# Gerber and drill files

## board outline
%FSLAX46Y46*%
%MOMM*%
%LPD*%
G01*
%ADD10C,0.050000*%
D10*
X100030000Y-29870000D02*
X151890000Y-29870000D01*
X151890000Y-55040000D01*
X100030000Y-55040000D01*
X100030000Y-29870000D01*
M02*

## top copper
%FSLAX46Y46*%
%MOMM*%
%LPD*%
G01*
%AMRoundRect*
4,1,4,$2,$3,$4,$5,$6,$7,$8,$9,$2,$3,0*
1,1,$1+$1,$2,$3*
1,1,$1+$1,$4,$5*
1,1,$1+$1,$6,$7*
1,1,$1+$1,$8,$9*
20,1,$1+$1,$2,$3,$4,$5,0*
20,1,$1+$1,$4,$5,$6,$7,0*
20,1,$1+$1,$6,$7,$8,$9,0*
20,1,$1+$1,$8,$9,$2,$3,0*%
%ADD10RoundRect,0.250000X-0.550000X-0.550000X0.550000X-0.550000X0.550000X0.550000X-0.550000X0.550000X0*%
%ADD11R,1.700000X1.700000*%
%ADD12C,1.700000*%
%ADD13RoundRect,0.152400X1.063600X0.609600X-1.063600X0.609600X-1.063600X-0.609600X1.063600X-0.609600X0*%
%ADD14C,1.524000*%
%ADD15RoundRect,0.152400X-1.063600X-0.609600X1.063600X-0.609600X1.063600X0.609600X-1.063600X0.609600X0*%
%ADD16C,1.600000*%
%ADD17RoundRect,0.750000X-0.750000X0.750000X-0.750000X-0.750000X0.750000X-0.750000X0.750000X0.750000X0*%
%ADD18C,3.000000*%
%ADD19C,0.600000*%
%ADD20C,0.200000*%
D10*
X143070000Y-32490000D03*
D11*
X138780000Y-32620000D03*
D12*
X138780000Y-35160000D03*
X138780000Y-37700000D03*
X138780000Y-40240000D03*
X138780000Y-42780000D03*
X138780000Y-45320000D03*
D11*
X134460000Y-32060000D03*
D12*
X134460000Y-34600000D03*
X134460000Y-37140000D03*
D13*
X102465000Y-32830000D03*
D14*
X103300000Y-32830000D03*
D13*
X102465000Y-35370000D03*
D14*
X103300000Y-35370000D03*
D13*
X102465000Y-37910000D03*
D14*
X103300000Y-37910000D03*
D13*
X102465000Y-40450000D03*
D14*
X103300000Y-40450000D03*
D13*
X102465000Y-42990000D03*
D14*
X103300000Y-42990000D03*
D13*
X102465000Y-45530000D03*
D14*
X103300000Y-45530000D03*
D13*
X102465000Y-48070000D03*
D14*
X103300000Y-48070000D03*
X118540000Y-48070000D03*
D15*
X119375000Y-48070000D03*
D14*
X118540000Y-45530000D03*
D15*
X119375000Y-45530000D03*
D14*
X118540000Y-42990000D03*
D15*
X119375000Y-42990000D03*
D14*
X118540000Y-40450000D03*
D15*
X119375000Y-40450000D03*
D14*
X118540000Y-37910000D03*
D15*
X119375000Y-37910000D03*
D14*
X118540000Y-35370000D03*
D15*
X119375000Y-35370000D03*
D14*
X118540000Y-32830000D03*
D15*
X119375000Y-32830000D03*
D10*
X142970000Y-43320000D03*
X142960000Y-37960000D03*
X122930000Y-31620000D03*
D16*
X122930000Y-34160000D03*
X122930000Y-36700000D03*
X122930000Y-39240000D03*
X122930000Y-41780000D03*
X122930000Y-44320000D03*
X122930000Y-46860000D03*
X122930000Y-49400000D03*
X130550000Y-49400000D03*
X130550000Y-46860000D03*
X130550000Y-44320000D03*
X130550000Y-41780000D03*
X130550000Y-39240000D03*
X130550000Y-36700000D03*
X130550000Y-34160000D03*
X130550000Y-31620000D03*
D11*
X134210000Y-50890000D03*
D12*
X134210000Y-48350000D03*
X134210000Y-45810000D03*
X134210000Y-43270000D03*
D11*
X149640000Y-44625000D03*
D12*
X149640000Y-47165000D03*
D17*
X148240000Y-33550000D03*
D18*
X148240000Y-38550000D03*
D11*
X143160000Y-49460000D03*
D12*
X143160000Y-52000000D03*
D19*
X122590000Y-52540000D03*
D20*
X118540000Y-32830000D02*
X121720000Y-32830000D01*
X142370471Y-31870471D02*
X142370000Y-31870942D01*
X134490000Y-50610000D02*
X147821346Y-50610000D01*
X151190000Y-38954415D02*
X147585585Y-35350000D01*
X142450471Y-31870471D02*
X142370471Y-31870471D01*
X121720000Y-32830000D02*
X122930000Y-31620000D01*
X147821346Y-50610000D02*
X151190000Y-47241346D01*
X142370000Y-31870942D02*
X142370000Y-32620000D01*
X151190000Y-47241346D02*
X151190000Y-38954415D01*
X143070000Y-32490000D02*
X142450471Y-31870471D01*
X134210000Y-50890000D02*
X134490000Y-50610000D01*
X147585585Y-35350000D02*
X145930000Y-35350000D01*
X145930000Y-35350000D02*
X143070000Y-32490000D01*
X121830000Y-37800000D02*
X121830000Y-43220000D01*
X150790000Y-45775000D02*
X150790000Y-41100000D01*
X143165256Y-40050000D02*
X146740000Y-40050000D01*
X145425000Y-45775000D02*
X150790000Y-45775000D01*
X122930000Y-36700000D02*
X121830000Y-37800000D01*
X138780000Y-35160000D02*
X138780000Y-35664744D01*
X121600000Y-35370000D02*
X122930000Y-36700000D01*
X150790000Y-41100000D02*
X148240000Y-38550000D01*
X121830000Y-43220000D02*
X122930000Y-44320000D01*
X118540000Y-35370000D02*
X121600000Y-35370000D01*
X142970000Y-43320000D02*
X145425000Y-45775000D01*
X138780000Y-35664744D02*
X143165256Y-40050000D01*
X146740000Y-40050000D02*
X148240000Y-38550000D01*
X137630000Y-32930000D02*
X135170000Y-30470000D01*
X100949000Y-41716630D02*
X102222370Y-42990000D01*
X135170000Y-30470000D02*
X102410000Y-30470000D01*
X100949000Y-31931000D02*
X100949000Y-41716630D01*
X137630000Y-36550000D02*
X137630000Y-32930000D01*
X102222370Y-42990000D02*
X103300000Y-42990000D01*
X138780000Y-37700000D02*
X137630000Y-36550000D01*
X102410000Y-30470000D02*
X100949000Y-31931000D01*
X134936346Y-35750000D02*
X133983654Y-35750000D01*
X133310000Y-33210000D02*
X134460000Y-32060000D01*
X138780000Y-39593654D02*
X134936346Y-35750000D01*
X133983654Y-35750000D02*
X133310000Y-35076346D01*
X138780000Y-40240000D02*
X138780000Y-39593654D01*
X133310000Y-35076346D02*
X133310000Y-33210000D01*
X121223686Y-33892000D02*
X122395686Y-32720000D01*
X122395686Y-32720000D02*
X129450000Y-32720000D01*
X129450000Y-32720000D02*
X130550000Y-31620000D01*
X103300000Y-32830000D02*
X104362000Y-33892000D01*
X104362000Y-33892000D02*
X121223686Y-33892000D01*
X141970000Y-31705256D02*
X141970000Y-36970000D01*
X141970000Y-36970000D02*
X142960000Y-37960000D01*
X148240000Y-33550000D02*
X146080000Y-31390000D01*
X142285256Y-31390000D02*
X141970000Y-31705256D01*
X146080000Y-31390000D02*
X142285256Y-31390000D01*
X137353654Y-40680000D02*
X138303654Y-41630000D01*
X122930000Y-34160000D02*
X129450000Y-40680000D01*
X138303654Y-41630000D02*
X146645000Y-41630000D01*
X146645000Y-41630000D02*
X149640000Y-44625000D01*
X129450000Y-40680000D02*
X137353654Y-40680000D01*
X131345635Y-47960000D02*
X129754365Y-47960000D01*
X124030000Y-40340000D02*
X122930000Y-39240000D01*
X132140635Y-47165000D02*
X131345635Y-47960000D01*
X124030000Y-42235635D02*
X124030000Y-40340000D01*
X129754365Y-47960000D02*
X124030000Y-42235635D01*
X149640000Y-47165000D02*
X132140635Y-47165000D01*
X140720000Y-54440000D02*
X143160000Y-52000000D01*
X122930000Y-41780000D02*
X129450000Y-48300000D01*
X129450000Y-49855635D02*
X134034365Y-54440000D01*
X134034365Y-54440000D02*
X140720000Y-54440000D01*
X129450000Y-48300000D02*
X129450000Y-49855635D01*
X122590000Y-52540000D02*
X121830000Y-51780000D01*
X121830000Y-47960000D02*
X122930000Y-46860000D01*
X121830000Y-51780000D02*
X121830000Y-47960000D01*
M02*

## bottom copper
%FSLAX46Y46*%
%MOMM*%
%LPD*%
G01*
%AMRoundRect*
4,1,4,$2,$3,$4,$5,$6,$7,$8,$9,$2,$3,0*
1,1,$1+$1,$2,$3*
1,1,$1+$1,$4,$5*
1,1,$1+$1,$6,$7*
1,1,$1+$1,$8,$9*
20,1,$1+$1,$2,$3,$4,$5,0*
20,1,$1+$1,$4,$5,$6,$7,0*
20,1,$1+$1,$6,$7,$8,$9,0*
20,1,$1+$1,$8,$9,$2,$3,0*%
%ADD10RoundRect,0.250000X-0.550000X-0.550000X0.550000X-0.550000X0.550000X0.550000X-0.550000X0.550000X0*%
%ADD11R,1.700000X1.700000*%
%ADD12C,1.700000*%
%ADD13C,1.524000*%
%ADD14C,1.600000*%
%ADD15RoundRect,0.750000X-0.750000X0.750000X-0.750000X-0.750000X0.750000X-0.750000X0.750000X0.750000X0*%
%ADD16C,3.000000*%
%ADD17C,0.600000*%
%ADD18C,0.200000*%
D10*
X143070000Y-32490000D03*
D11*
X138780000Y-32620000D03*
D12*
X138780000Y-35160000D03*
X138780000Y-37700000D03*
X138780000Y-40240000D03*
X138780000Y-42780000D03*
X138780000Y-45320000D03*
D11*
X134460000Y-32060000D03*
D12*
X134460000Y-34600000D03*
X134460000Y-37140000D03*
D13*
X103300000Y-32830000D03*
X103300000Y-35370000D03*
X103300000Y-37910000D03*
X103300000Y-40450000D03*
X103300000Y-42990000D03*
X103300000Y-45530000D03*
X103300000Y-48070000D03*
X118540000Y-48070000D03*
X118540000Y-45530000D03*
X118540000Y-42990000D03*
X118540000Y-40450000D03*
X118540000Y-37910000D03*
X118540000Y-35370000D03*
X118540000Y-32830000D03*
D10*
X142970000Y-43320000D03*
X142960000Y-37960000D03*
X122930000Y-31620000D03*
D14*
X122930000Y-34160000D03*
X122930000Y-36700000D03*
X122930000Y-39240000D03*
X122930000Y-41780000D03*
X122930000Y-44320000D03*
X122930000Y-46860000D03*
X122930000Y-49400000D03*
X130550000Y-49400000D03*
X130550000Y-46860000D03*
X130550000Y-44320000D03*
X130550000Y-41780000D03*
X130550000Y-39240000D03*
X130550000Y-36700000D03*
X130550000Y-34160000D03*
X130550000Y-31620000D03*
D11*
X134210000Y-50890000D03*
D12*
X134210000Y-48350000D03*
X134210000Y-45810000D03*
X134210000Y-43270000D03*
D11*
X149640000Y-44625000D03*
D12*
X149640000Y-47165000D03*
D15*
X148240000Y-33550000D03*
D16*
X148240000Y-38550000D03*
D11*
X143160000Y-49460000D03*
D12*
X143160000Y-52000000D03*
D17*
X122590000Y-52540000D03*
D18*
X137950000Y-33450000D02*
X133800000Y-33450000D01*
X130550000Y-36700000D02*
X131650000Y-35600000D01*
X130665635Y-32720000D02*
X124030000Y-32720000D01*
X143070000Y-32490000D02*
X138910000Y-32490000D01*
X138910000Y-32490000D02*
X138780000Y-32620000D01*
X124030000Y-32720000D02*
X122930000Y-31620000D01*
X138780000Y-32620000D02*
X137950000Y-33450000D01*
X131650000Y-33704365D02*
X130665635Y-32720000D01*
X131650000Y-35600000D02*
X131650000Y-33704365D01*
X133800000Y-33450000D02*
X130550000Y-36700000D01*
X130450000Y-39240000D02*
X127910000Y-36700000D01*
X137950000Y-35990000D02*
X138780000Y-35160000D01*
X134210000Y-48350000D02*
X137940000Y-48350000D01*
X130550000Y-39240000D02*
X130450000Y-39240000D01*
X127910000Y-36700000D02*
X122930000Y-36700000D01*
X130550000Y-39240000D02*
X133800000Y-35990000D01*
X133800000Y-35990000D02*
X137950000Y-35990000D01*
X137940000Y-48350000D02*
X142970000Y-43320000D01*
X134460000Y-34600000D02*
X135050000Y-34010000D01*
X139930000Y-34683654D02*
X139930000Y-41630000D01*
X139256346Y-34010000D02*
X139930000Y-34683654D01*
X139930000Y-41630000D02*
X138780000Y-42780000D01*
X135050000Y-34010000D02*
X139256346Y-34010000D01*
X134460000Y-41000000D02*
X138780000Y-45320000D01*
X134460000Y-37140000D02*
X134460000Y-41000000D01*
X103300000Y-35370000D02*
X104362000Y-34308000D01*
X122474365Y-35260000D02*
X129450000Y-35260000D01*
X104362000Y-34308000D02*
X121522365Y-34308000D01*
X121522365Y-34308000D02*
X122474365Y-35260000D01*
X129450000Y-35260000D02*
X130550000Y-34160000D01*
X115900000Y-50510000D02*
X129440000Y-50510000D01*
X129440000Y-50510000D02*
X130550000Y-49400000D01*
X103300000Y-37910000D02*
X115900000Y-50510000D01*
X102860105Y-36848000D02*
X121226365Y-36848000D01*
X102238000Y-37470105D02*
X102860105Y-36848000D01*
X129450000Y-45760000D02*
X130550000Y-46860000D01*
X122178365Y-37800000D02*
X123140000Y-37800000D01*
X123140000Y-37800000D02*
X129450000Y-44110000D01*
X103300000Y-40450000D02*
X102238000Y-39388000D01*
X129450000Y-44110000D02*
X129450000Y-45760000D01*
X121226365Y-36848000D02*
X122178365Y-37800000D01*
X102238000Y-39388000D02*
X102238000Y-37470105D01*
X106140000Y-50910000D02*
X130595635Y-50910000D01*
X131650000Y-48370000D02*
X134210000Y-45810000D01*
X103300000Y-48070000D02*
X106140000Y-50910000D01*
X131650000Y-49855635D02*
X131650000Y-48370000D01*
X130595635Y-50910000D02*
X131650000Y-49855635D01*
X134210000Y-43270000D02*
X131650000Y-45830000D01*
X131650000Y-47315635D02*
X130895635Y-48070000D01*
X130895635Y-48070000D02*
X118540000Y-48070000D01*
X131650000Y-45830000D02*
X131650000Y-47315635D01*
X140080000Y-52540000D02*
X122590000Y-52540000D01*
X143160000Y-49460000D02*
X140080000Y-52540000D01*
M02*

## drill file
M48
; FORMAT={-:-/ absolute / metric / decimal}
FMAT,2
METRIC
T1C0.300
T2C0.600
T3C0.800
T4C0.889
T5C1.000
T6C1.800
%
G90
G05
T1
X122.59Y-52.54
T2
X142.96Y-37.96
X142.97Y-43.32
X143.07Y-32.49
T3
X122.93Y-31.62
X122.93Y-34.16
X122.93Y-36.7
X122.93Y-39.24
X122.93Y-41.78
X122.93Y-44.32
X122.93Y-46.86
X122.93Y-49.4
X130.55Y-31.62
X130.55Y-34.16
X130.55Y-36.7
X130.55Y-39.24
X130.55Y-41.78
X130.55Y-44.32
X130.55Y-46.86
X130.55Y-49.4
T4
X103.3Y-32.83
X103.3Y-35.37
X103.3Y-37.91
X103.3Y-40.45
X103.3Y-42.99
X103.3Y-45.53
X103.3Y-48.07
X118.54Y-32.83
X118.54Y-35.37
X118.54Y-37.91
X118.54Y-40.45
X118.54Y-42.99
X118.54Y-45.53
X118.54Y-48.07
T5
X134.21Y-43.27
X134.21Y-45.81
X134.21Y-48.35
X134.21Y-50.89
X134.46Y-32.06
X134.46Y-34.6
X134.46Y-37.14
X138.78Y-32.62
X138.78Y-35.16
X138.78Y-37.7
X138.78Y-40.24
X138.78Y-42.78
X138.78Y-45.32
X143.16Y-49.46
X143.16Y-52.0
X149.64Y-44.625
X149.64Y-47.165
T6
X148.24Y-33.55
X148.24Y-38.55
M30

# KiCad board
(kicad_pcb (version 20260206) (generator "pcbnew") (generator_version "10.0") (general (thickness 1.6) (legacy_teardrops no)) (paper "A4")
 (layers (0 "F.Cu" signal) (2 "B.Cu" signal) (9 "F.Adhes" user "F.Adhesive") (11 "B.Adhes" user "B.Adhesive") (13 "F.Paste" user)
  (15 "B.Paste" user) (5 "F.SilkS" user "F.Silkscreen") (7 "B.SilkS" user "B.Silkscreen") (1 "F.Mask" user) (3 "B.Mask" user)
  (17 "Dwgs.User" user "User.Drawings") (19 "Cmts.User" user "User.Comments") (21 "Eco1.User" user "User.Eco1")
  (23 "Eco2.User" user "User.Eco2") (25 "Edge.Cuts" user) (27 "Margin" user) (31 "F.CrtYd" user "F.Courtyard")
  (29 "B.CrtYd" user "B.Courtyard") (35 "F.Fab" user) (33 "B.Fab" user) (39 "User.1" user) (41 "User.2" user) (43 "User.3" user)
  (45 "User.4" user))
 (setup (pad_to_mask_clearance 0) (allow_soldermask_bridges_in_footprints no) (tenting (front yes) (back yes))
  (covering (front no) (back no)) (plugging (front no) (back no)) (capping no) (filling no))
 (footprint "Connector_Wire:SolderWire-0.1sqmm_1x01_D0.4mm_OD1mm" (layer "F.Cu") (at 143.07 32.49)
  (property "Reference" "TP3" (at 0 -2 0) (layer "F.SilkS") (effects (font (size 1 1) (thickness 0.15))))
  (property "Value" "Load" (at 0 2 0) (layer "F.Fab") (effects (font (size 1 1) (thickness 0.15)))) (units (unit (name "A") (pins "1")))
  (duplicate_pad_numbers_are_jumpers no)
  (pad "1" thru_hole roundrect (at 0 0) (size 1.6 1.6) (drill 0.6) (layers "*.Cu" "*.Mask") (remove_unused_layers no)
   (roundrect_rratio 0.15625) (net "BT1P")))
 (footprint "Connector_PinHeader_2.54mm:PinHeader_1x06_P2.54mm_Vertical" (layer "F.Cu") (at 138.78 32.62)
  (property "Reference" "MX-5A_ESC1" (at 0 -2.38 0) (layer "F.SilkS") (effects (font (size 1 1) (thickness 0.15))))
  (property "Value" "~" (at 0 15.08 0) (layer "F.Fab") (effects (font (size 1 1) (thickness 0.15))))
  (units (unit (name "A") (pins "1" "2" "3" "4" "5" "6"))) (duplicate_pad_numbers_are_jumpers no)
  (pad "1" thru_hole rect (at 0 0) (size 1.7 1.7) (drill 1) (layers "*.Cu" "*.Mask") (remove_unused_layers no) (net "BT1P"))
  (pad "2" thru_hole circle (at 0 2.54) (size 1.7 1.7) (drill 1) (layers "*.Cu" "*.Mask") (remove_unused_layers no) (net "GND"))
  (pad "3" thru_hole circle (at 0 5.08) (size 1.7 1.7) (drill 1) (layers "*.Cu" "*.Mask") (remove_unused_layers no)
   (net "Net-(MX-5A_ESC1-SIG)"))
  (pad "4" thru_hole circle (at 0 7.62) (size 1.7 1.7) (drill 1) (layers "*.Cu" "*.Mask") (remove_unused_layers no)
   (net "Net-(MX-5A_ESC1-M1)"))
  (pad "5" thru_hole circle (at 0 10.16) (size 1.7 1.7) (drill 1) (layers "*.Cu" "*.Mask") (remove_unused_layers no)
   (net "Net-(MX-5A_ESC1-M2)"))
  (pad "6" thru_hole circle (at 0 12.7) (size 1.7 1.7) (drill 1) (layers "*.Cu" "*.Mask") (remove_unused_layers no)
   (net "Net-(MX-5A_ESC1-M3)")))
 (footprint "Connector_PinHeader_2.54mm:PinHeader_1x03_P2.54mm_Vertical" (layer "F.Cu") (at 134.46 32.06)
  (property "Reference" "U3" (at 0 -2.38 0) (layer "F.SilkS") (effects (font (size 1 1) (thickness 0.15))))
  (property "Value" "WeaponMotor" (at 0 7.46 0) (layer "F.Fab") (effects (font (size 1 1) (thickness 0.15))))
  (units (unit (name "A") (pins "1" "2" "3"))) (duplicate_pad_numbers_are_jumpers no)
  (pad "1" thru_hole rect (at 0 0) (size 1.7 1.7) (drill 1) (layers "*.Cu" "*.Mask") (remove_unused_layers no) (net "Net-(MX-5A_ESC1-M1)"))
  (pad "2" thru_hole circle (at 0 2.54) (size 1.7 1.7) (drill 1) (layers "*.Cu" "*.Mask") (remove_unused_layers no)
   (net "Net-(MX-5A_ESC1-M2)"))
  (pad "3" thru_hole circle (at 0 5.08) (size 1.7 1.7) (drill 1) (layers "*.Cu" "*.Mask") (remove_unused_layers no)
   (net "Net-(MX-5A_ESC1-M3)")))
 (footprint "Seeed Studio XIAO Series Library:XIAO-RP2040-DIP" (layer "F.Cu") (at 110.92 40.45)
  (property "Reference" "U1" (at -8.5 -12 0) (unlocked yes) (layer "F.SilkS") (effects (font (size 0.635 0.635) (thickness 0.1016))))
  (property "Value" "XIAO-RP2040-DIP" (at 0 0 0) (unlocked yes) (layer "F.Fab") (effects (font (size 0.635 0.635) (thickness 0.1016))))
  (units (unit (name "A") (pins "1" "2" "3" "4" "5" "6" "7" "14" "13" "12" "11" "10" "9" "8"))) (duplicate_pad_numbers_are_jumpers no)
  (pad "1" smd roundrect (at -8.455 -7.62 180) (size 2.432 1.524) (layers "F.Cu" "F.Mask") (roundrect_rratio 0.1) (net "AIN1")
   (thermal_bridge_angle 45))
  (pad "1" thru_hole circle (at -7.62 -7.62 180) (size 1.524 1.524) (drill 0.889) (layers "*.Cu" "*.Mask") (remove_unused_layers no)
   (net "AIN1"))
  (pad "2" smd roundrect (at -8.455 -5.08 180) (size 2.432 1.524) (layers "F.Cu" "F.Mask") (roundrect_rratio 0.1) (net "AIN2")
   (thermal_bridge_angle 45))
  (pad "2" thru_hole circle (at -7.62 -5.08 180) (size 1.524 1.524) (drill 0.889) (layers "*.Cu" "*.Mask") (remove_unused_layers no)
   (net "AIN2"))
  (pad "3" smd roundrect (at -8.455 -2.54 180) (size 2.432 1.524) (layers "F.Cu" "F.Mask") (roundrect_rratio 0.1) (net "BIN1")
   (thermal_bridge_angle 45))
  (pad "3" thru_hole circle (at -7.62 -2.54 180) (size 1.524 1.524) (drill 0.889) (layers "*.Cu" "*.Mask") (remove_unused_layers no)
   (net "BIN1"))
  (pad "4" smd roundrect (at -8.455 0 180) (size 2.432 1.524) (layers "F.Cu" "F.Mask") (roundrect_rratio 0.1) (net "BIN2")
   (thermal_bridge_angle 45))
  (pad "4" thru_hole circle (at -7.62 0 180) (size 1.524 1.524) (drill 0.889) (layers "*.Cu" "*.Mask") (remove_unused_layers no)
   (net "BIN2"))
  (pad "5" smd roundrect (at -8.455 2.54 180) (size 2.432 1.524) (layers "F.Cu" "F.Mask") (roundrect_rratio 0.1)
   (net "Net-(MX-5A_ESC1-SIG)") (thermal_bridge_angle 45))
  (pad "5" thru_hole circle (at -7.62 2.54 180) (size 1.524 1.524) (drill 0.889) (layers "*.Cu" "*.Mask") (remove_unused_layers no)
   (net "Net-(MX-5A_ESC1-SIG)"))
  (pad "6" smd roundrect (at -8.455 5.08 180) (size 2.432 1.524) (layers "F.Cu" "F.Mask") (roundrect_rratio 0.1)
   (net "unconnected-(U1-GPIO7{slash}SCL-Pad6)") (thermal_bridge_angle 45))
  (pad "6" thru_hole circle (at -7.62 5.08 180) (size 1.524 1.524) (drill 0.889) (layers "*.Cu" "*.Mask") (remove_unused_layers no)
   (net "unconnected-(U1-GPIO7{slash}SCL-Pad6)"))
  (pad "7" smd roundrect (at -8.455 7.62 180) (size 2.432 1.524) (layers "F.Cu" "F.Mask") (roundrect_rratio 0.1)
   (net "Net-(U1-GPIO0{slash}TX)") (thermal_bridge_angle 45))
  (pad "7" thru_hole circle (at -7.62 7.62 180) (size 1.524 1.524) (drill 0.889) (layers "*.Cu" "*.Mask") (remove_unused_layers no)
   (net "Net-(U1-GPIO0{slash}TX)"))
  (pad "8" thru_hole circle (at 7.62 7.62) (size 1.524 1.524) (drill 0.889) (layers "*.Cu" "*.Mask") (remove_unused_layers no)
   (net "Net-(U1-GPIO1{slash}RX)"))
  (pad "8" smd roundrect (at 8.455 7.62) (size 2.432 1.524) (layers "F.Cu" "F.Mask") (roundrect_rratio 0.1) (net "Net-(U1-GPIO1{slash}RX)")
   (thermal_bridge_angle 45))
  (pad "9" thru_hole circle (at 7.62 5.08) (size 1.524 1.524) (drill 0.889) (layers "*.Cu" "*.Mask") (remove_unused_layers no)
   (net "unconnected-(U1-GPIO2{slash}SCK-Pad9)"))
  (pad "9" smd roundrect (at 8.455 5.08) (size 2.432 1.524) (layers "F.Cu" "F.Mask") (roundrect_rratio 0.1)
   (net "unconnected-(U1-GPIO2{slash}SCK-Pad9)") (thermal_bridge_angle 45))
  (pad "10" thru_hole circle (at 7.62 2.54) (size 1.524 1.524) (drill 0.889) (layers "*.Cu" "*.Mask") (remove_unused_layers no)
   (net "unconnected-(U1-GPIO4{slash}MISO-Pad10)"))
  (pad "10" smd roundrect (at 8.455 2.54) (size 2.432 1.524) (layers "F.Cu" "F.Mask") (roundrect_rratio 0.1)
   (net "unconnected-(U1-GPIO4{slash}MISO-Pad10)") (thermal_bridge_angle 45))
  (pad "11" thru_hole circle (at 7.62 0) (size 1.524 1.524) (drill 0.889) (layers "*.Cu" "*.Mask") (remove_unused_layers no)
   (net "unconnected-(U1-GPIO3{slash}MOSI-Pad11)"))
  (pad "11" smd roundrect (at 8.455 0) (size 2.432 1.524) (layers "F.Cu" "F.Mask") (roundrect_rratio 0.1)
   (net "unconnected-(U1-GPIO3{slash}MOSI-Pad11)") (thermal_bridge_angle 45))
  (pad "12" thru_hole circle (at 7.62 -2.54) (size 1.524 1.524) (drill 0.889) (layers "*.Cu" "*.Mask") (remove_unused_layers no)
   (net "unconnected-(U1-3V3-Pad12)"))
  (pad "12" smd roundrect (at 8.455 -2.54) (size 2.432 1.524) (layers "F.Cu" "F.Mask") (roundrect_rratio 0.1)
   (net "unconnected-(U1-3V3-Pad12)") (thermal_bridge_angle 45))
  (pad "13" thru_hole circle (at 7.62 -5.08) (size 1.524 1.524) (drill 0.889) (layers "*.Cu" "*.Mask") (remove_unused_layers no) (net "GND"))
  (pad "13" smd roundrect (at 8.455 -5.08) (size 2.432 1.524) (layers "F.Cu" "F.Mask") (roundrect_rratio 0.1) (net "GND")
   (thermal_bridge_angle 45))
  (pad "14" thru_hole circle (at 7.62 -7.62) (size 1.524 1.524) (drill 0.889) (layers "*.Cu" "*.Mask") (remove_unused_layers no)
   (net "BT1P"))
  (pad "14" smd roundrect (at 8.455 -7.62) (size 2.432 1.524) (layers "F.Cu" "F.Mask") (roundrect_rratio 0.1) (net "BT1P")
   (thermal_bridge_angle 45)))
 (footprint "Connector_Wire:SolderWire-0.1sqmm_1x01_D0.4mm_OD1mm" (layer "F.Cu") (at 142.97 43.32)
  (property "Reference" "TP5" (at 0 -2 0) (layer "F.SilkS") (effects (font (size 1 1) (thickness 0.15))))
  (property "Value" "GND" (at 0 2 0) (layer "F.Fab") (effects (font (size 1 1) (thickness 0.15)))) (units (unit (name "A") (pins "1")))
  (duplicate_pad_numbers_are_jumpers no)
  (pad "1" thru_hole roundrect (at 0 0) (size 1.6 1.6) (drill 0.6) (layers "*.Cu" "*.Mask") (remove_unused_layers no)
   (roundrect_rratio 0.15625) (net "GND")))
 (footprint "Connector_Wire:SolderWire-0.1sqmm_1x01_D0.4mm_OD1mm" (layer "F.Cu") (at 142.96 37.96)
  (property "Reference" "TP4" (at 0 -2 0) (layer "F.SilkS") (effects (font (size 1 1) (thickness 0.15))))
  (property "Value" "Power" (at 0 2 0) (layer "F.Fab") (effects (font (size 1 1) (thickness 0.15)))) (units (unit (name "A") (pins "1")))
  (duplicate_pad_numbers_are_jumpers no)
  (pad "1" thru_hole roundrect (at 0 0) (size 1.6 1.6) (drill 0.6) (layers "*.Cu" "*.Mask") (remove_unused_layers no)
   (roundrect_rratio 0.15625) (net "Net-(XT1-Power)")))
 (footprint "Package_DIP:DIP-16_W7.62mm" (layer "F.Cu") (at 122.93 31.62)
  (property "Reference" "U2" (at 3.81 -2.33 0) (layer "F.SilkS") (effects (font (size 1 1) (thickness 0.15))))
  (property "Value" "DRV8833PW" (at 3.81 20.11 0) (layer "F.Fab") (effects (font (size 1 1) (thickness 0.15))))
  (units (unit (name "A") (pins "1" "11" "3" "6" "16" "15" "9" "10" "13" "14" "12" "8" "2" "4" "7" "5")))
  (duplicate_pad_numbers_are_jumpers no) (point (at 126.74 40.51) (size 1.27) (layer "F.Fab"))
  (pad "1" thru_hole roundrect (at 0 0) (size 1.6 1.6) (drill 0.8) (layers "*.Cu" "*.Mask") (remove_unused_layers no)
   (roundrect_rratio 0.15625) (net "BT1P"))
  (pad "2" thru_hole circle (at 0 2.54) (size 1.6 1.6) (drill 0.8) (layers "*.Cu" "*.Mask") (remove_unused_layers no) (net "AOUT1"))
  (pad "3" thru_hole circle (at 0 5.08) (size 1.6 1.6) (drill 0.8) (layers "*.Cu" "*.Mask") (remove_unused_layers no) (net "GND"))
  (pad "4" thru_hole circle (at 0 7.62) (size 1.6 1.6) (drill 0.8) (layers "*.Cu" "*.Mask") (remove_unused_layers no) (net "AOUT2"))
  (pad "5" thru_hole circle (at 0 10.16) (size 1.6 1.6) (drill 0.8) (layers "*.Cu" "*.Mask") (remove_unused_layers no) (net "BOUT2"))
  (pad "6" thru_hole circle (at 0 12.7) (size 1.6 1.6) (drill 0.8) (layers "*.Cu" "*.Mask") (remove_unused_layers no) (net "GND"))
  (pad "7" thru_hole circle (at 0 15.24) (size 1.6 1.6) (drill 0.8) (layers "*.Cu" "*.Mask") (remove_unused_layers no) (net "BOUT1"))
  (pad "8" thru_hole circle (at 0 17.78) (size 1.6 1.6) (drill 0.8) (layers "*.Cu" "*.Mask") (remove_unused_layers no)
   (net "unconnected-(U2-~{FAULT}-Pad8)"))
  (pad "9" thru_hole circle (at 7.62 17.78) (size 1.6 1.6) (drill 0.8) (layers "*.Cu" "*.Mask") (remove_unused_layers no) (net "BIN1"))
  (pad "10" thru_hole circle (at 7.62 15.24) (size 1.6 1.6) (drill 0.8) (layers "*.Cu" "*.Mask") (remove_unused_layers no) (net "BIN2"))
  (pad "11" thru_hole circle (at 7.62 12.7) (size 1.6 1.6) (drill 0.8) (layers "*.Cu" "*.Mask") (remove_unused_layers no)
   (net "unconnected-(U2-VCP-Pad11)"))
  (pad "12" thru_hole circle (at 7.62 10.16) (size 1.6 1.6) (drill 0.8) (layers "*.Cu" "*.Mask") (remove_unused_layers no)
   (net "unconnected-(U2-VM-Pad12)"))
  (pad "13" thru_hole circle (at 7.62 7.62) (size 1.6 1.6) (drill 0.8) (layers "*.Cu" "*.Mask") (remove_unused_layers no) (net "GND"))
  (pad "14" thru_hole circle (at 7.62 5.08) (size 1.6 1.6) (drill 0.8) (layers "*.Cu" "*.Mask") (remove_unused_layers no) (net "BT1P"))
  (pad "15" thru_hole circle (at 7.62 2.54) (size 1.6 1.6) (drill 0.8) (layers "*.Cu" "*.Mask") (remove_unused_layers no) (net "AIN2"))
  (pad "16" thru_hole circle (at 7.62 0) (size 1.6 1.6) (drill 0.8) (layers "*.Cu" "*.Mask") (remove_unused_layers no) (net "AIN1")))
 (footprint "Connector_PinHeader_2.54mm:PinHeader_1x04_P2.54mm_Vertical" (layer "F.Cu") (at 134.21 50.89 180)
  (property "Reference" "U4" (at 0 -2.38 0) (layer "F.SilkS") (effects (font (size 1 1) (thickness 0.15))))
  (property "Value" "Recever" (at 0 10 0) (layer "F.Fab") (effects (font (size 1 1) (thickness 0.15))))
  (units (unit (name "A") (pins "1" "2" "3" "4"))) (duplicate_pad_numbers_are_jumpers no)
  (pad "1" thru_hole rect (at 0 0 180) (size 1.7 1.7) (drill 1) (layers "*.Cu" "*.Mask") (remove_unused_layers no) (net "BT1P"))
  (pad "2" thru_hole circle (at 0 2.54 180) (size 1.7 1.7) (drill 1) (layers "*.Cu" "*.Mask") (remove_unused_layers no) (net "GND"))
  (pad "3" thru_hole circle (at 0 5.08 180) (size 1.7 1.7) (drill 1) (layers "*.Cu" "*.Mask") (remove_unused_layers no)
   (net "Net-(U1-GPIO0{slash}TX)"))
  (pad "4" thru_hole circle (at 0 7.62 180) (size 1.7 1.7) (drill 1) (layers "*.Cu" "*.Mask") (remove_unused_layers no)
   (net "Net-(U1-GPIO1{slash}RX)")))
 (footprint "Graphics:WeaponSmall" (layer "F.Cu") (at 100.447555 49.76791)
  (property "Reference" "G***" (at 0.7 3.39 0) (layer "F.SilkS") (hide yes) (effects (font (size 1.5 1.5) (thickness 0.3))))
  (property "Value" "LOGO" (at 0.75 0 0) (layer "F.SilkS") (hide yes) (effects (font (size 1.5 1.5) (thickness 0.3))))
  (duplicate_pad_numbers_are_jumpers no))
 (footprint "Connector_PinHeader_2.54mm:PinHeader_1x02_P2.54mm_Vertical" (layer "F.Cu") (at 149.64 44.625)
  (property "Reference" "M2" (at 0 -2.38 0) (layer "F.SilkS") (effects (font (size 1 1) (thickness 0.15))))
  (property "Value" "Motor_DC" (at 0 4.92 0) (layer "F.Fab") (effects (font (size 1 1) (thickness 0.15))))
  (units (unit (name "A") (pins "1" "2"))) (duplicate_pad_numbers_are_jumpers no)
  (pad "1" thru_hole rect (at 0 0) (size 1.7 1.7) (drill 1) (layers "*.Cu" "*.Mask") (remove_unused_layers no) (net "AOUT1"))
  (pad "2" thru_hole circle (at 0 2.54) (size 1.7 1.7) (drill 1) (layers "*.Cu" "*.Mask") (remove_unused_layers no) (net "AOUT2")))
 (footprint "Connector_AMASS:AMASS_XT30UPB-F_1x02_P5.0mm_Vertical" (layer "F.Cu") (at 148.24 33.55 -90)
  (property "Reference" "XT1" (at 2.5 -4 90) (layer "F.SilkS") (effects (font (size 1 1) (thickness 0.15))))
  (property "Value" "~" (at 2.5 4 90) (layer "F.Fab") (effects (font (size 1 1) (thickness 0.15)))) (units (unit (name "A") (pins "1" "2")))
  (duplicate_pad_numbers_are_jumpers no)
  (pad "1" thru_hole roundrect (at 0 0 270) (size 3 3) (drill 1.8) (layers "*.Cu" "*.Mask") (remove_unused_layers no)
   (roundrect_rratio 0.25) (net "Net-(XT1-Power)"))
  (pad "2" thru_hole circle (at 5 0 270) (size 3 3) (drill 1.8) (layers "*.Cu" "*.Mask") (remove_unused_layers no) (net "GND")))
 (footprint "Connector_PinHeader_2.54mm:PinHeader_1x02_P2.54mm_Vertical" (layer "F.Cu") (at 143.16 49.46)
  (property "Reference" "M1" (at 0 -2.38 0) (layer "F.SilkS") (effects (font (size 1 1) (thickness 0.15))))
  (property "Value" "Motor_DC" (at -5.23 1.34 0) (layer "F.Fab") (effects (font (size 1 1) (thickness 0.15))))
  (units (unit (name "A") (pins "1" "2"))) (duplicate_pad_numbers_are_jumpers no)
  (pad "1" thru_hole rect (at 0 0) (size 1.7 1.7) (drill 1) (layers "*.Cu" "*.Mask") (remove_unused_layers no) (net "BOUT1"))
  (pad "2" thru_hole circle (at 0 2.54) (size 1.7 1.7) (drill 1) (layers "*.Cu" "*.Mask") (remove_unused_layers no) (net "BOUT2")))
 (gr_rect (start 100.03 29.87) (end 151.89 55.04) (stroke (width 0.05) (type default)) (fill no) (layer "Edge.Cuts"))
 (segment (start 118.54 32.83) (end 121.72 32.83) (width 0.2) (layer "F.Cu") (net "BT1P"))
 (segment (start 142.370471 31.870471) (end 142.37 31.870942) (width 0.2) (layer "F.Cu") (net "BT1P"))
 (segment (start 134.49 50.61) (end 147.821346 50.61) (width 0.2) (layer "F.Cu") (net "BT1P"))
 (segment (start 151.19 38.954415) (end 147.585585 35.35) (width 0.2) (layer "F.Cu") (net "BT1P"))
 (segment (start 142.450471 31.870471) (end 142.370471 31.870471) (width 0.2) (layer "F.Cu") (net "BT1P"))
 (segment (start 121.72 32.83) (end 122.93 31.62) (width 0.2) (layer "F.Cu") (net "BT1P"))
 (segment (start 147.821346 50.61) (end 151.19 47.241346) (width 0.2) (layer "F.Cu") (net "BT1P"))
 (segment (start 142.37 31.870942) (end 142.37 32.62) (width 0.2) (layer "F.Cu") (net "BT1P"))
 (segment (start 151.19 47.241346) (end 151.19 38.954415) (width 0.2) (layer "F.Cu") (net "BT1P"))
 (segment (start 143.07 32.49) (end 142.450471 31.870471) (width 0.2) (layer "F.Cu") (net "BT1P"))
 (segment (start 134.21 50.89) (end 134.49 50.61) (width 0.2) (layer "F.Cu") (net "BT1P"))
 (segment (start 147.585585 35.35) (end 145.93 35.35) (width 0.2) (layer "F.Cu") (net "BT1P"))
 (segment (start 145.93 35.35) (end 143.07 32.49) (width 0.2) (layer "F.Cu") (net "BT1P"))
 (segment (start 137.95 33.45) (end 133.8 33.45) (width 0.2) (layer "B.Cu") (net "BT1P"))
 (segment (start 130.55 36.7) (end 131.65 35.6) (width 0.2) (layer "B.Cu") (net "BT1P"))
 (segment (start 130.665635 32.72) (end 124.03 32.72) (width 0.2) (layer "B.Cu") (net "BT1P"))
 (segment (start 143.07 32.49) (end 138.91 32.49) (width 0.2) (layer "B.Cu") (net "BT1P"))
 (segment (start 138.91 32.49) (end 138.78 32.62) (width 0.2) (layer "B.Cu") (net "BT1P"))
 (segment (start 124.03 32.72) (end 122.93 31.62) (width 0.2) (layer "B.Cu") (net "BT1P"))
 (segment (start 138.78 32.62) (end 137.95 33.45) (width 0.2) (layer "B.Cu") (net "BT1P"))
 (segment (start 131.65 33.704365) (end 130.665635 32.72) (width 0.2) (layer "B.Cu") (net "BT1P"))
 (segment (start 131.65 35.6) (end 131.65 33.704365) (width 0.2) (layer "B.Cu") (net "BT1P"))
 (segment (start 133.8 33.45) (end 130.55 36.7) (width 0.2) (layer "B.Cu") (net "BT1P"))
 (segment (start 121.83 37.8) (end 121.83 43.22) (width 0.2) (layer "F.Cu") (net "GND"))
 (segment (start 150.79 45.775) (end 150.79 41.1) (width 0.2) (layer "F.Cu") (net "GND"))
 (segment (start 143.165256 40.05) (end 146.74 40.05) (width 0.2) (layer "F.Cu") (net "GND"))
 (segment (start 145.425 45.775) (end 150.79 45.775) (width 0.2) (layer "F.Cu") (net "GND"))
 (segment (start 122.93 36.7) (end 121.83 37.8) (width 0.2) (layer "F.Cu") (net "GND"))
 (segment (start 138.78 35.16) (end 138.78 35.664744) (width 0.2) (layer "F.Cu") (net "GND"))
 (segment (start 121.6 35.37) (end 122.93 36.7) (width 0.2) (layer "F.Cu") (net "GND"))
 (segment (start 150.79 41.1) (end 148.24 38.55) (width 0.2) (layer "F.Cu") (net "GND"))
 (segment (start 121.83 43.22) (end 122.93 44.32) (width 0.2) (layer "F.Cu") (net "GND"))
 (segment (start 118.54 35.37) (end 121.6 35.37) (width 0.2) (layer "F.Cu") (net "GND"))
 (segment (start 142.97 43.32) (end 145.425 45.775) (width 0.2) (layer "F.Cu") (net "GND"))
 (segment (start 138.78 35.664744) (end 143.165256 40.05) (width 0.2) (layer "F.Cu") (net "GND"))
 (segment (start 146.74 40.05) (end 148.24 38.55) (width 0.2) (layer "F.Cu") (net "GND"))
 (segment (start 130.45 39.24) (end 127.91 36.7) (width 0.2) (layer "B.Cu") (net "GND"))
 (segment (start 137.95 35.99) (end 138.78 35.16) (width 0.2) (layer "B.Cu") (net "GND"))
 (segment (start 134.21 48.35) (end 137.94 48.35) (width 0.2) (layer "B.Cu") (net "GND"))
 (segment (start 130.55 39.24) (end 130.45 39.24) (width 0.2) (layer "B.Cu") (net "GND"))
 (segment (start 127.91 36.7) (end 122.93 36.7) (width 0.2) (layer "B.Cu") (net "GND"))
 (segment (start 130.55 39.24) (end 133.8 35.99) (width 0.2) (layer "B.Cu") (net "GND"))
 (segment (start 133.8 35.99) (end 137.95 35.99) (width 0.2) (layer "B.Cu") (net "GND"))
 (segment (start 137.94 48.35) (end 142.97 43.32) (width 0.2) (layer "B.Cu") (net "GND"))
 (segment (start 137.63 32.93) (end 135.17 30.47) (width 0.2) (layer "F.Cu") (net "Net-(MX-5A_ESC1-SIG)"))
 (segment (start 100.949 41.71663) (end 102.22237 42.99) (width 0.2) (layer "F.Cu") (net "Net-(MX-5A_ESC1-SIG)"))
 (segment (start 135.17 30.47) (end 102.41 30.47) (width 0.2) (layer "F.Cu") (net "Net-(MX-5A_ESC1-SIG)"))
 (segment (start 100.949 31.931) (end 100.949 41.71663) (width 0.2) (layer "F.Cu") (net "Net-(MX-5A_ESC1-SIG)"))
 (segment (start 137.63 36.55) (end 137.63 32.93) (width 0.2) (layer "F.Cu") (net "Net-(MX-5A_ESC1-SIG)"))
 (segment (start 102.22237 42.99) (end 103.3 42.99) (width 0.2) (layer "F.Cu") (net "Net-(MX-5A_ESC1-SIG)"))
 (segment (start 138.78 37.7) (end 137.63 36.55) (width 0.2) (layer "F.Cu") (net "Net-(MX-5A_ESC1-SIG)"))
 (segment (start 102.41 30.47) (end 100.949 31.931) (width 0.2) (layer "F.Cu") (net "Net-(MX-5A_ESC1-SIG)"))
 (segment (start 134.936346 35.75) (end 133.983654 35.75) (width 0.2) (layer "F.Cu") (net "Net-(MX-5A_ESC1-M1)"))
 (segment (start 133.31 33.21) (end 134.46 32.06) (width 0.2) (layer "F.Cu") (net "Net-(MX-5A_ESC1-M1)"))
 (segment (start 138.78 39.593654) (end 134.936346 35.75) (width 0.2) (layer "F.Cu") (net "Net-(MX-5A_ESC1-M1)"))
 (segment (start 133.983654 35.75) (end 133.31 35.076346) (width 0.2) (layer "F.Cu") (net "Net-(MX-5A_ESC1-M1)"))
 (segment (start 138.78 40.24) (end 138.78 39.593654) (width 0.2) (layer "F.Cu") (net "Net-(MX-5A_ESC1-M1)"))
 (segment (start 133.31 35.076346) (end 133.31 33.21) (width 0.2) (layer "F.Cu") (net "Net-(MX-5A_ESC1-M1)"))
 (segment (start 134.46 34.6) (end 135.05 34.01) (width 0.2) (layer "B.Cu") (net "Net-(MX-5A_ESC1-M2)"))
 (segment (start 139.93 34.683654) (end 139.93 41.63) (width 0.2) (layer "B.Cu") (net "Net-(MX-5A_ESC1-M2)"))
 (segment (start 139.256346 34.01) (end 139.93 34.683654) (width 0.2) (layer "B.Cu") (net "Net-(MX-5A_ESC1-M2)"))
 (segment (start 139.93 41.63) (end 138.78 42.78) (width 0.2) (layer "B.Cu") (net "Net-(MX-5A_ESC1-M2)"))
 (segment (start 135.05 34.01) (end 139.256346 34.01) (width 0.2) (layer "B.Cu") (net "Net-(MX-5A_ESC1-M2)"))
 (segment (start 134.46 41) (end 138.78 45.32) (width 0.2) (layer "B.Cu") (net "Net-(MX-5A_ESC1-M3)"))
 (segment (start 134.46 37.14) (end 134.46 41) (width 0.2) (layer "B.Cu") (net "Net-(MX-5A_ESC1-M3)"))
 (segment (start 121.223686 33.892) (end 122.395686 32.72) (width 0.2) (layer "F.Cu") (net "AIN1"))
 (segment (start 122.395686 32.72) (end 129.45 32.72) (width 0.2) (layer "F.Cu") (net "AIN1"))
 (segment (start 129.45 32.72) (end 130.55 31.62) (width 0.2) (layer "F.Cu") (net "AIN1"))
 (segment (start 103.3 32.83) (end 104.362 33.892) (width 0.2) (layer "F.Cu") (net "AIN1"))
 (segment (start 104.362 33.892) (end 121.223686 33.892) (width 0.2) (layer "F.Cu") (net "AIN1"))
 (segment (start 103.3 35.37) (end 104.362 34.308) (width 0.2) (layer "B.Cu") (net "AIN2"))
 (segment (start 122.474365 35.26) (end 129.45 35.26) (width 0.2) (layer "B.Cu") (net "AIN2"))
 (segment (start 104.362 34.308) (end 121.522365 34.308) (width 0.2) (layer "B.Cu") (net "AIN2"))
 (segment (start 121.522365 34.308) (end 122.474365 35.26) (width 0.2) (layer "B.Cu") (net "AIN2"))
 (segment (start 129.45 35.26) (end 130.55 34.16) (width 0.2) (layer "B.Cu") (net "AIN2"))
 (segment (start 115.9 50.51) (end 129.44 50.51) (width 0.2) (layer "B.Cu") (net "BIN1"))
 (segment (start 129.44 50.51) (end 130.55 49.4) (width 0.2) (layer "B.Cu") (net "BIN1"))
 (segment (start 103.3 37.91) (end 115.9 50.51) (width 0.2) (layer "B.Cu") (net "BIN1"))
 (segment (start 102.860105 36.848) (end 121.226365 36.848) (width 0.2) (layer "B.Cu") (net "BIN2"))
 (segment (start 102.238 37.470105) (end 102.860105 36.848) (width 0.2) (layer "B.Cu") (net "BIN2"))
 (segment (start 129.45 45.76) (end 130.55 46.86) (width 0.2) (layer "B.Cu") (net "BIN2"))
 (segment (start 122.178365 37.8) (end 123.14 37.8) (width 0.2) (layer "B.Cu") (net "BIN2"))
 (segment (start 123.14 37.8) (end 129.45 44.11) (width 0.2) (layer "B.Cu") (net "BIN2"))
 (segment (start 103.3 40.45) (end 102.238 39.388) (width 0.2) (layer "B.Cu") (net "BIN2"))
 (segment (start 129.45 44.11) (end 129.45 45.76) (width 0.2) (layer "B.Cu") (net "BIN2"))
 (segment (start 121.226365 36.848) (end 122.178365 37.8) (width 0.2) (layer "B.Cu") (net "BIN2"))
 (segment (start 102.238 39.388) (end 102.238 37.470105) (width 0.2) (layer "B.Cu") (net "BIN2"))
 (segment (start 106.14 50.91) (end 130.595635 50.91) (width 0.2) (layer "B.Cu") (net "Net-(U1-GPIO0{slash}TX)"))
 (segment (start 131.65 48.37) (end 134.21 45.81) (width 0.2) (layer "B.Cu") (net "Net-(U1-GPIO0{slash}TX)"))
 (segment (start 103.3 48.07) (end 106.14 50.91) (width 0.2) (layer "B.Cu") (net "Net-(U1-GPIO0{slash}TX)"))
 (segment (start 131.65 49.855635) (end 131.65 48.37) (width 0.2) (layer "B.Cu") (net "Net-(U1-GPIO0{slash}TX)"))
 (segment (start 130.595635 50.91) (end 131.65 49.855635) (width 0.2) (layer "B.Cu") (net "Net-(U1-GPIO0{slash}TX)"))
 (segment (start 134.21 43.27) (end 131.65 45.83) (width 0.2) (layer "B.Cu") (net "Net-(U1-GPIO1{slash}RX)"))
 (segment (start 131.65 47.315635) (end 130.895635 48.07) (width 0.2) (layer "B.Cu") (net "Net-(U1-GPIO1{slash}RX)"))
 (segment (start 130.895635 48.07) (end 118.54 48.07) (width 0.2) (layer "B.Cu") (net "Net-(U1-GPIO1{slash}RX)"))
 (segment (start 131.65 45.83) (end 131.65 47.315635) (width 0.2) (layer "B.Cu") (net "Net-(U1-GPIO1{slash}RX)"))
 (segment (start 141.97 31.705256) (end 141.97 36.97) (width 0.2) (layer "F.Cu") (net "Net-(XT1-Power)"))
 (segment (start 141.97 36.97) (end 142.96 37.96) (width 0.2) (layer "F.Cu") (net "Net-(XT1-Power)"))
 (segment (start 148.24 33.55) (end 146.08 31.39) (width 0.2) (layer "F.Cu") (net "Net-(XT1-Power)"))
 (segment (start 142.285256 31.39) (end 141.97 31.705256) (width 0.2) (layer "F.Cu") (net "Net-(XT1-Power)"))
 (segment (start 146.08 31.39) (end 142.285256 31.39) (width 0.2) (layer "F.Cu") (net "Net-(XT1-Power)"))
 (segment (start 137.353654 40.68) (end 138.303654 41.63) (width 0.2) (layer "F.Cu") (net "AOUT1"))
 (segment (start 122.93 34.16) (end 129.45 40.68) (width 0.2) (layer "F.Cu") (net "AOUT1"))
 (segment (start 138.303654 41.63) (end 146.645 41.63) (width 0.2) (layer "F.Cu") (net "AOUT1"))
 (segment (start 146.645 41.63) (end 149.64 44.625) (width 0.2) (layer "F.Cu") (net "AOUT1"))
 (segment (start 129.45 40.68) (end 137.353654 40.68) (width 0.2) (layer "F.Cu") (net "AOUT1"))
 (segment (start 131.345635 47.96) (end 129.754365 47.96) (width 0.2) (layer "F.Cu") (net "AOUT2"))
 (segment (start 124.03 40.34) (end 122.93 39.24) (width 0.2) (layer "F.Cu") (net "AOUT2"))
 (segment (start 132.140635 47.165) (end 131.345635 47.96) (width 0.2) (layer "F.Cu") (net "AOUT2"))
 (segment (start 124.03 42.235635) (end 124.03 40.34) (width 0.2) (layer "F.Cu") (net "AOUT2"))
 (segment (start 129.754365 47.96) (end 124.03 42.235635) (width 0.2) (layer "F.Cu") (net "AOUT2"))
 (segment (start 149.64 47.165) (end 132.140635 47.165) (width 0.2) (layer "F.Cu") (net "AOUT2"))
 (segment (start 140.72 54.44) (end 143.16 52) (width 0.2) (layer "F.Cu") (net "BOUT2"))
 (segment (start 122.93 41.78) (end 129.45 48.3) (width 0.2) (layer "F.Cu") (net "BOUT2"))
 (segment (start 129.45 49.855635) (end 134.034365 54.44) (width 0.2) (layer "F.Cu") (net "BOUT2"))
 (segment (start 134.034365 54.44) (end 140.72 54.44) (width 0.2) (layer "F.Cu") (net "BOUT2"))
 (segment (start 129.45 48.3) (end 129.45 49.855635) (width 0.2) (layer "F.Cu") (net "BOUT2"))
 (segment (start 122.59 52.54) (end 121.83 51.78) (width 0.2) (layer "F.Cu") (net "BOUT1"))
 (segment (start 121.83 47.96) (end 122.93 46.86) (width 0.2) (layer "F.Cu") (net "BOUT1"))
 (segment (start 121.83 51.78) (end 121.83 47.96) (width 0.2) (layer "F.Cu") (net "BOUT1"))
 (via (at 122.59 52.54) (size 0.6) (drill 0.3) (layers "F.Cu" "B.Cu") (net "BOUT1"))
 (segment (start 140.08 52.54) (end 122.59 52.54) (width 0.2) (layer "B.Cu") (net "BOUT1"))
 (segment (start 143.16 49.46) (end 140.08 52.54) (width 0.2) (layer "B.Cu") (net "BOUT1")))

